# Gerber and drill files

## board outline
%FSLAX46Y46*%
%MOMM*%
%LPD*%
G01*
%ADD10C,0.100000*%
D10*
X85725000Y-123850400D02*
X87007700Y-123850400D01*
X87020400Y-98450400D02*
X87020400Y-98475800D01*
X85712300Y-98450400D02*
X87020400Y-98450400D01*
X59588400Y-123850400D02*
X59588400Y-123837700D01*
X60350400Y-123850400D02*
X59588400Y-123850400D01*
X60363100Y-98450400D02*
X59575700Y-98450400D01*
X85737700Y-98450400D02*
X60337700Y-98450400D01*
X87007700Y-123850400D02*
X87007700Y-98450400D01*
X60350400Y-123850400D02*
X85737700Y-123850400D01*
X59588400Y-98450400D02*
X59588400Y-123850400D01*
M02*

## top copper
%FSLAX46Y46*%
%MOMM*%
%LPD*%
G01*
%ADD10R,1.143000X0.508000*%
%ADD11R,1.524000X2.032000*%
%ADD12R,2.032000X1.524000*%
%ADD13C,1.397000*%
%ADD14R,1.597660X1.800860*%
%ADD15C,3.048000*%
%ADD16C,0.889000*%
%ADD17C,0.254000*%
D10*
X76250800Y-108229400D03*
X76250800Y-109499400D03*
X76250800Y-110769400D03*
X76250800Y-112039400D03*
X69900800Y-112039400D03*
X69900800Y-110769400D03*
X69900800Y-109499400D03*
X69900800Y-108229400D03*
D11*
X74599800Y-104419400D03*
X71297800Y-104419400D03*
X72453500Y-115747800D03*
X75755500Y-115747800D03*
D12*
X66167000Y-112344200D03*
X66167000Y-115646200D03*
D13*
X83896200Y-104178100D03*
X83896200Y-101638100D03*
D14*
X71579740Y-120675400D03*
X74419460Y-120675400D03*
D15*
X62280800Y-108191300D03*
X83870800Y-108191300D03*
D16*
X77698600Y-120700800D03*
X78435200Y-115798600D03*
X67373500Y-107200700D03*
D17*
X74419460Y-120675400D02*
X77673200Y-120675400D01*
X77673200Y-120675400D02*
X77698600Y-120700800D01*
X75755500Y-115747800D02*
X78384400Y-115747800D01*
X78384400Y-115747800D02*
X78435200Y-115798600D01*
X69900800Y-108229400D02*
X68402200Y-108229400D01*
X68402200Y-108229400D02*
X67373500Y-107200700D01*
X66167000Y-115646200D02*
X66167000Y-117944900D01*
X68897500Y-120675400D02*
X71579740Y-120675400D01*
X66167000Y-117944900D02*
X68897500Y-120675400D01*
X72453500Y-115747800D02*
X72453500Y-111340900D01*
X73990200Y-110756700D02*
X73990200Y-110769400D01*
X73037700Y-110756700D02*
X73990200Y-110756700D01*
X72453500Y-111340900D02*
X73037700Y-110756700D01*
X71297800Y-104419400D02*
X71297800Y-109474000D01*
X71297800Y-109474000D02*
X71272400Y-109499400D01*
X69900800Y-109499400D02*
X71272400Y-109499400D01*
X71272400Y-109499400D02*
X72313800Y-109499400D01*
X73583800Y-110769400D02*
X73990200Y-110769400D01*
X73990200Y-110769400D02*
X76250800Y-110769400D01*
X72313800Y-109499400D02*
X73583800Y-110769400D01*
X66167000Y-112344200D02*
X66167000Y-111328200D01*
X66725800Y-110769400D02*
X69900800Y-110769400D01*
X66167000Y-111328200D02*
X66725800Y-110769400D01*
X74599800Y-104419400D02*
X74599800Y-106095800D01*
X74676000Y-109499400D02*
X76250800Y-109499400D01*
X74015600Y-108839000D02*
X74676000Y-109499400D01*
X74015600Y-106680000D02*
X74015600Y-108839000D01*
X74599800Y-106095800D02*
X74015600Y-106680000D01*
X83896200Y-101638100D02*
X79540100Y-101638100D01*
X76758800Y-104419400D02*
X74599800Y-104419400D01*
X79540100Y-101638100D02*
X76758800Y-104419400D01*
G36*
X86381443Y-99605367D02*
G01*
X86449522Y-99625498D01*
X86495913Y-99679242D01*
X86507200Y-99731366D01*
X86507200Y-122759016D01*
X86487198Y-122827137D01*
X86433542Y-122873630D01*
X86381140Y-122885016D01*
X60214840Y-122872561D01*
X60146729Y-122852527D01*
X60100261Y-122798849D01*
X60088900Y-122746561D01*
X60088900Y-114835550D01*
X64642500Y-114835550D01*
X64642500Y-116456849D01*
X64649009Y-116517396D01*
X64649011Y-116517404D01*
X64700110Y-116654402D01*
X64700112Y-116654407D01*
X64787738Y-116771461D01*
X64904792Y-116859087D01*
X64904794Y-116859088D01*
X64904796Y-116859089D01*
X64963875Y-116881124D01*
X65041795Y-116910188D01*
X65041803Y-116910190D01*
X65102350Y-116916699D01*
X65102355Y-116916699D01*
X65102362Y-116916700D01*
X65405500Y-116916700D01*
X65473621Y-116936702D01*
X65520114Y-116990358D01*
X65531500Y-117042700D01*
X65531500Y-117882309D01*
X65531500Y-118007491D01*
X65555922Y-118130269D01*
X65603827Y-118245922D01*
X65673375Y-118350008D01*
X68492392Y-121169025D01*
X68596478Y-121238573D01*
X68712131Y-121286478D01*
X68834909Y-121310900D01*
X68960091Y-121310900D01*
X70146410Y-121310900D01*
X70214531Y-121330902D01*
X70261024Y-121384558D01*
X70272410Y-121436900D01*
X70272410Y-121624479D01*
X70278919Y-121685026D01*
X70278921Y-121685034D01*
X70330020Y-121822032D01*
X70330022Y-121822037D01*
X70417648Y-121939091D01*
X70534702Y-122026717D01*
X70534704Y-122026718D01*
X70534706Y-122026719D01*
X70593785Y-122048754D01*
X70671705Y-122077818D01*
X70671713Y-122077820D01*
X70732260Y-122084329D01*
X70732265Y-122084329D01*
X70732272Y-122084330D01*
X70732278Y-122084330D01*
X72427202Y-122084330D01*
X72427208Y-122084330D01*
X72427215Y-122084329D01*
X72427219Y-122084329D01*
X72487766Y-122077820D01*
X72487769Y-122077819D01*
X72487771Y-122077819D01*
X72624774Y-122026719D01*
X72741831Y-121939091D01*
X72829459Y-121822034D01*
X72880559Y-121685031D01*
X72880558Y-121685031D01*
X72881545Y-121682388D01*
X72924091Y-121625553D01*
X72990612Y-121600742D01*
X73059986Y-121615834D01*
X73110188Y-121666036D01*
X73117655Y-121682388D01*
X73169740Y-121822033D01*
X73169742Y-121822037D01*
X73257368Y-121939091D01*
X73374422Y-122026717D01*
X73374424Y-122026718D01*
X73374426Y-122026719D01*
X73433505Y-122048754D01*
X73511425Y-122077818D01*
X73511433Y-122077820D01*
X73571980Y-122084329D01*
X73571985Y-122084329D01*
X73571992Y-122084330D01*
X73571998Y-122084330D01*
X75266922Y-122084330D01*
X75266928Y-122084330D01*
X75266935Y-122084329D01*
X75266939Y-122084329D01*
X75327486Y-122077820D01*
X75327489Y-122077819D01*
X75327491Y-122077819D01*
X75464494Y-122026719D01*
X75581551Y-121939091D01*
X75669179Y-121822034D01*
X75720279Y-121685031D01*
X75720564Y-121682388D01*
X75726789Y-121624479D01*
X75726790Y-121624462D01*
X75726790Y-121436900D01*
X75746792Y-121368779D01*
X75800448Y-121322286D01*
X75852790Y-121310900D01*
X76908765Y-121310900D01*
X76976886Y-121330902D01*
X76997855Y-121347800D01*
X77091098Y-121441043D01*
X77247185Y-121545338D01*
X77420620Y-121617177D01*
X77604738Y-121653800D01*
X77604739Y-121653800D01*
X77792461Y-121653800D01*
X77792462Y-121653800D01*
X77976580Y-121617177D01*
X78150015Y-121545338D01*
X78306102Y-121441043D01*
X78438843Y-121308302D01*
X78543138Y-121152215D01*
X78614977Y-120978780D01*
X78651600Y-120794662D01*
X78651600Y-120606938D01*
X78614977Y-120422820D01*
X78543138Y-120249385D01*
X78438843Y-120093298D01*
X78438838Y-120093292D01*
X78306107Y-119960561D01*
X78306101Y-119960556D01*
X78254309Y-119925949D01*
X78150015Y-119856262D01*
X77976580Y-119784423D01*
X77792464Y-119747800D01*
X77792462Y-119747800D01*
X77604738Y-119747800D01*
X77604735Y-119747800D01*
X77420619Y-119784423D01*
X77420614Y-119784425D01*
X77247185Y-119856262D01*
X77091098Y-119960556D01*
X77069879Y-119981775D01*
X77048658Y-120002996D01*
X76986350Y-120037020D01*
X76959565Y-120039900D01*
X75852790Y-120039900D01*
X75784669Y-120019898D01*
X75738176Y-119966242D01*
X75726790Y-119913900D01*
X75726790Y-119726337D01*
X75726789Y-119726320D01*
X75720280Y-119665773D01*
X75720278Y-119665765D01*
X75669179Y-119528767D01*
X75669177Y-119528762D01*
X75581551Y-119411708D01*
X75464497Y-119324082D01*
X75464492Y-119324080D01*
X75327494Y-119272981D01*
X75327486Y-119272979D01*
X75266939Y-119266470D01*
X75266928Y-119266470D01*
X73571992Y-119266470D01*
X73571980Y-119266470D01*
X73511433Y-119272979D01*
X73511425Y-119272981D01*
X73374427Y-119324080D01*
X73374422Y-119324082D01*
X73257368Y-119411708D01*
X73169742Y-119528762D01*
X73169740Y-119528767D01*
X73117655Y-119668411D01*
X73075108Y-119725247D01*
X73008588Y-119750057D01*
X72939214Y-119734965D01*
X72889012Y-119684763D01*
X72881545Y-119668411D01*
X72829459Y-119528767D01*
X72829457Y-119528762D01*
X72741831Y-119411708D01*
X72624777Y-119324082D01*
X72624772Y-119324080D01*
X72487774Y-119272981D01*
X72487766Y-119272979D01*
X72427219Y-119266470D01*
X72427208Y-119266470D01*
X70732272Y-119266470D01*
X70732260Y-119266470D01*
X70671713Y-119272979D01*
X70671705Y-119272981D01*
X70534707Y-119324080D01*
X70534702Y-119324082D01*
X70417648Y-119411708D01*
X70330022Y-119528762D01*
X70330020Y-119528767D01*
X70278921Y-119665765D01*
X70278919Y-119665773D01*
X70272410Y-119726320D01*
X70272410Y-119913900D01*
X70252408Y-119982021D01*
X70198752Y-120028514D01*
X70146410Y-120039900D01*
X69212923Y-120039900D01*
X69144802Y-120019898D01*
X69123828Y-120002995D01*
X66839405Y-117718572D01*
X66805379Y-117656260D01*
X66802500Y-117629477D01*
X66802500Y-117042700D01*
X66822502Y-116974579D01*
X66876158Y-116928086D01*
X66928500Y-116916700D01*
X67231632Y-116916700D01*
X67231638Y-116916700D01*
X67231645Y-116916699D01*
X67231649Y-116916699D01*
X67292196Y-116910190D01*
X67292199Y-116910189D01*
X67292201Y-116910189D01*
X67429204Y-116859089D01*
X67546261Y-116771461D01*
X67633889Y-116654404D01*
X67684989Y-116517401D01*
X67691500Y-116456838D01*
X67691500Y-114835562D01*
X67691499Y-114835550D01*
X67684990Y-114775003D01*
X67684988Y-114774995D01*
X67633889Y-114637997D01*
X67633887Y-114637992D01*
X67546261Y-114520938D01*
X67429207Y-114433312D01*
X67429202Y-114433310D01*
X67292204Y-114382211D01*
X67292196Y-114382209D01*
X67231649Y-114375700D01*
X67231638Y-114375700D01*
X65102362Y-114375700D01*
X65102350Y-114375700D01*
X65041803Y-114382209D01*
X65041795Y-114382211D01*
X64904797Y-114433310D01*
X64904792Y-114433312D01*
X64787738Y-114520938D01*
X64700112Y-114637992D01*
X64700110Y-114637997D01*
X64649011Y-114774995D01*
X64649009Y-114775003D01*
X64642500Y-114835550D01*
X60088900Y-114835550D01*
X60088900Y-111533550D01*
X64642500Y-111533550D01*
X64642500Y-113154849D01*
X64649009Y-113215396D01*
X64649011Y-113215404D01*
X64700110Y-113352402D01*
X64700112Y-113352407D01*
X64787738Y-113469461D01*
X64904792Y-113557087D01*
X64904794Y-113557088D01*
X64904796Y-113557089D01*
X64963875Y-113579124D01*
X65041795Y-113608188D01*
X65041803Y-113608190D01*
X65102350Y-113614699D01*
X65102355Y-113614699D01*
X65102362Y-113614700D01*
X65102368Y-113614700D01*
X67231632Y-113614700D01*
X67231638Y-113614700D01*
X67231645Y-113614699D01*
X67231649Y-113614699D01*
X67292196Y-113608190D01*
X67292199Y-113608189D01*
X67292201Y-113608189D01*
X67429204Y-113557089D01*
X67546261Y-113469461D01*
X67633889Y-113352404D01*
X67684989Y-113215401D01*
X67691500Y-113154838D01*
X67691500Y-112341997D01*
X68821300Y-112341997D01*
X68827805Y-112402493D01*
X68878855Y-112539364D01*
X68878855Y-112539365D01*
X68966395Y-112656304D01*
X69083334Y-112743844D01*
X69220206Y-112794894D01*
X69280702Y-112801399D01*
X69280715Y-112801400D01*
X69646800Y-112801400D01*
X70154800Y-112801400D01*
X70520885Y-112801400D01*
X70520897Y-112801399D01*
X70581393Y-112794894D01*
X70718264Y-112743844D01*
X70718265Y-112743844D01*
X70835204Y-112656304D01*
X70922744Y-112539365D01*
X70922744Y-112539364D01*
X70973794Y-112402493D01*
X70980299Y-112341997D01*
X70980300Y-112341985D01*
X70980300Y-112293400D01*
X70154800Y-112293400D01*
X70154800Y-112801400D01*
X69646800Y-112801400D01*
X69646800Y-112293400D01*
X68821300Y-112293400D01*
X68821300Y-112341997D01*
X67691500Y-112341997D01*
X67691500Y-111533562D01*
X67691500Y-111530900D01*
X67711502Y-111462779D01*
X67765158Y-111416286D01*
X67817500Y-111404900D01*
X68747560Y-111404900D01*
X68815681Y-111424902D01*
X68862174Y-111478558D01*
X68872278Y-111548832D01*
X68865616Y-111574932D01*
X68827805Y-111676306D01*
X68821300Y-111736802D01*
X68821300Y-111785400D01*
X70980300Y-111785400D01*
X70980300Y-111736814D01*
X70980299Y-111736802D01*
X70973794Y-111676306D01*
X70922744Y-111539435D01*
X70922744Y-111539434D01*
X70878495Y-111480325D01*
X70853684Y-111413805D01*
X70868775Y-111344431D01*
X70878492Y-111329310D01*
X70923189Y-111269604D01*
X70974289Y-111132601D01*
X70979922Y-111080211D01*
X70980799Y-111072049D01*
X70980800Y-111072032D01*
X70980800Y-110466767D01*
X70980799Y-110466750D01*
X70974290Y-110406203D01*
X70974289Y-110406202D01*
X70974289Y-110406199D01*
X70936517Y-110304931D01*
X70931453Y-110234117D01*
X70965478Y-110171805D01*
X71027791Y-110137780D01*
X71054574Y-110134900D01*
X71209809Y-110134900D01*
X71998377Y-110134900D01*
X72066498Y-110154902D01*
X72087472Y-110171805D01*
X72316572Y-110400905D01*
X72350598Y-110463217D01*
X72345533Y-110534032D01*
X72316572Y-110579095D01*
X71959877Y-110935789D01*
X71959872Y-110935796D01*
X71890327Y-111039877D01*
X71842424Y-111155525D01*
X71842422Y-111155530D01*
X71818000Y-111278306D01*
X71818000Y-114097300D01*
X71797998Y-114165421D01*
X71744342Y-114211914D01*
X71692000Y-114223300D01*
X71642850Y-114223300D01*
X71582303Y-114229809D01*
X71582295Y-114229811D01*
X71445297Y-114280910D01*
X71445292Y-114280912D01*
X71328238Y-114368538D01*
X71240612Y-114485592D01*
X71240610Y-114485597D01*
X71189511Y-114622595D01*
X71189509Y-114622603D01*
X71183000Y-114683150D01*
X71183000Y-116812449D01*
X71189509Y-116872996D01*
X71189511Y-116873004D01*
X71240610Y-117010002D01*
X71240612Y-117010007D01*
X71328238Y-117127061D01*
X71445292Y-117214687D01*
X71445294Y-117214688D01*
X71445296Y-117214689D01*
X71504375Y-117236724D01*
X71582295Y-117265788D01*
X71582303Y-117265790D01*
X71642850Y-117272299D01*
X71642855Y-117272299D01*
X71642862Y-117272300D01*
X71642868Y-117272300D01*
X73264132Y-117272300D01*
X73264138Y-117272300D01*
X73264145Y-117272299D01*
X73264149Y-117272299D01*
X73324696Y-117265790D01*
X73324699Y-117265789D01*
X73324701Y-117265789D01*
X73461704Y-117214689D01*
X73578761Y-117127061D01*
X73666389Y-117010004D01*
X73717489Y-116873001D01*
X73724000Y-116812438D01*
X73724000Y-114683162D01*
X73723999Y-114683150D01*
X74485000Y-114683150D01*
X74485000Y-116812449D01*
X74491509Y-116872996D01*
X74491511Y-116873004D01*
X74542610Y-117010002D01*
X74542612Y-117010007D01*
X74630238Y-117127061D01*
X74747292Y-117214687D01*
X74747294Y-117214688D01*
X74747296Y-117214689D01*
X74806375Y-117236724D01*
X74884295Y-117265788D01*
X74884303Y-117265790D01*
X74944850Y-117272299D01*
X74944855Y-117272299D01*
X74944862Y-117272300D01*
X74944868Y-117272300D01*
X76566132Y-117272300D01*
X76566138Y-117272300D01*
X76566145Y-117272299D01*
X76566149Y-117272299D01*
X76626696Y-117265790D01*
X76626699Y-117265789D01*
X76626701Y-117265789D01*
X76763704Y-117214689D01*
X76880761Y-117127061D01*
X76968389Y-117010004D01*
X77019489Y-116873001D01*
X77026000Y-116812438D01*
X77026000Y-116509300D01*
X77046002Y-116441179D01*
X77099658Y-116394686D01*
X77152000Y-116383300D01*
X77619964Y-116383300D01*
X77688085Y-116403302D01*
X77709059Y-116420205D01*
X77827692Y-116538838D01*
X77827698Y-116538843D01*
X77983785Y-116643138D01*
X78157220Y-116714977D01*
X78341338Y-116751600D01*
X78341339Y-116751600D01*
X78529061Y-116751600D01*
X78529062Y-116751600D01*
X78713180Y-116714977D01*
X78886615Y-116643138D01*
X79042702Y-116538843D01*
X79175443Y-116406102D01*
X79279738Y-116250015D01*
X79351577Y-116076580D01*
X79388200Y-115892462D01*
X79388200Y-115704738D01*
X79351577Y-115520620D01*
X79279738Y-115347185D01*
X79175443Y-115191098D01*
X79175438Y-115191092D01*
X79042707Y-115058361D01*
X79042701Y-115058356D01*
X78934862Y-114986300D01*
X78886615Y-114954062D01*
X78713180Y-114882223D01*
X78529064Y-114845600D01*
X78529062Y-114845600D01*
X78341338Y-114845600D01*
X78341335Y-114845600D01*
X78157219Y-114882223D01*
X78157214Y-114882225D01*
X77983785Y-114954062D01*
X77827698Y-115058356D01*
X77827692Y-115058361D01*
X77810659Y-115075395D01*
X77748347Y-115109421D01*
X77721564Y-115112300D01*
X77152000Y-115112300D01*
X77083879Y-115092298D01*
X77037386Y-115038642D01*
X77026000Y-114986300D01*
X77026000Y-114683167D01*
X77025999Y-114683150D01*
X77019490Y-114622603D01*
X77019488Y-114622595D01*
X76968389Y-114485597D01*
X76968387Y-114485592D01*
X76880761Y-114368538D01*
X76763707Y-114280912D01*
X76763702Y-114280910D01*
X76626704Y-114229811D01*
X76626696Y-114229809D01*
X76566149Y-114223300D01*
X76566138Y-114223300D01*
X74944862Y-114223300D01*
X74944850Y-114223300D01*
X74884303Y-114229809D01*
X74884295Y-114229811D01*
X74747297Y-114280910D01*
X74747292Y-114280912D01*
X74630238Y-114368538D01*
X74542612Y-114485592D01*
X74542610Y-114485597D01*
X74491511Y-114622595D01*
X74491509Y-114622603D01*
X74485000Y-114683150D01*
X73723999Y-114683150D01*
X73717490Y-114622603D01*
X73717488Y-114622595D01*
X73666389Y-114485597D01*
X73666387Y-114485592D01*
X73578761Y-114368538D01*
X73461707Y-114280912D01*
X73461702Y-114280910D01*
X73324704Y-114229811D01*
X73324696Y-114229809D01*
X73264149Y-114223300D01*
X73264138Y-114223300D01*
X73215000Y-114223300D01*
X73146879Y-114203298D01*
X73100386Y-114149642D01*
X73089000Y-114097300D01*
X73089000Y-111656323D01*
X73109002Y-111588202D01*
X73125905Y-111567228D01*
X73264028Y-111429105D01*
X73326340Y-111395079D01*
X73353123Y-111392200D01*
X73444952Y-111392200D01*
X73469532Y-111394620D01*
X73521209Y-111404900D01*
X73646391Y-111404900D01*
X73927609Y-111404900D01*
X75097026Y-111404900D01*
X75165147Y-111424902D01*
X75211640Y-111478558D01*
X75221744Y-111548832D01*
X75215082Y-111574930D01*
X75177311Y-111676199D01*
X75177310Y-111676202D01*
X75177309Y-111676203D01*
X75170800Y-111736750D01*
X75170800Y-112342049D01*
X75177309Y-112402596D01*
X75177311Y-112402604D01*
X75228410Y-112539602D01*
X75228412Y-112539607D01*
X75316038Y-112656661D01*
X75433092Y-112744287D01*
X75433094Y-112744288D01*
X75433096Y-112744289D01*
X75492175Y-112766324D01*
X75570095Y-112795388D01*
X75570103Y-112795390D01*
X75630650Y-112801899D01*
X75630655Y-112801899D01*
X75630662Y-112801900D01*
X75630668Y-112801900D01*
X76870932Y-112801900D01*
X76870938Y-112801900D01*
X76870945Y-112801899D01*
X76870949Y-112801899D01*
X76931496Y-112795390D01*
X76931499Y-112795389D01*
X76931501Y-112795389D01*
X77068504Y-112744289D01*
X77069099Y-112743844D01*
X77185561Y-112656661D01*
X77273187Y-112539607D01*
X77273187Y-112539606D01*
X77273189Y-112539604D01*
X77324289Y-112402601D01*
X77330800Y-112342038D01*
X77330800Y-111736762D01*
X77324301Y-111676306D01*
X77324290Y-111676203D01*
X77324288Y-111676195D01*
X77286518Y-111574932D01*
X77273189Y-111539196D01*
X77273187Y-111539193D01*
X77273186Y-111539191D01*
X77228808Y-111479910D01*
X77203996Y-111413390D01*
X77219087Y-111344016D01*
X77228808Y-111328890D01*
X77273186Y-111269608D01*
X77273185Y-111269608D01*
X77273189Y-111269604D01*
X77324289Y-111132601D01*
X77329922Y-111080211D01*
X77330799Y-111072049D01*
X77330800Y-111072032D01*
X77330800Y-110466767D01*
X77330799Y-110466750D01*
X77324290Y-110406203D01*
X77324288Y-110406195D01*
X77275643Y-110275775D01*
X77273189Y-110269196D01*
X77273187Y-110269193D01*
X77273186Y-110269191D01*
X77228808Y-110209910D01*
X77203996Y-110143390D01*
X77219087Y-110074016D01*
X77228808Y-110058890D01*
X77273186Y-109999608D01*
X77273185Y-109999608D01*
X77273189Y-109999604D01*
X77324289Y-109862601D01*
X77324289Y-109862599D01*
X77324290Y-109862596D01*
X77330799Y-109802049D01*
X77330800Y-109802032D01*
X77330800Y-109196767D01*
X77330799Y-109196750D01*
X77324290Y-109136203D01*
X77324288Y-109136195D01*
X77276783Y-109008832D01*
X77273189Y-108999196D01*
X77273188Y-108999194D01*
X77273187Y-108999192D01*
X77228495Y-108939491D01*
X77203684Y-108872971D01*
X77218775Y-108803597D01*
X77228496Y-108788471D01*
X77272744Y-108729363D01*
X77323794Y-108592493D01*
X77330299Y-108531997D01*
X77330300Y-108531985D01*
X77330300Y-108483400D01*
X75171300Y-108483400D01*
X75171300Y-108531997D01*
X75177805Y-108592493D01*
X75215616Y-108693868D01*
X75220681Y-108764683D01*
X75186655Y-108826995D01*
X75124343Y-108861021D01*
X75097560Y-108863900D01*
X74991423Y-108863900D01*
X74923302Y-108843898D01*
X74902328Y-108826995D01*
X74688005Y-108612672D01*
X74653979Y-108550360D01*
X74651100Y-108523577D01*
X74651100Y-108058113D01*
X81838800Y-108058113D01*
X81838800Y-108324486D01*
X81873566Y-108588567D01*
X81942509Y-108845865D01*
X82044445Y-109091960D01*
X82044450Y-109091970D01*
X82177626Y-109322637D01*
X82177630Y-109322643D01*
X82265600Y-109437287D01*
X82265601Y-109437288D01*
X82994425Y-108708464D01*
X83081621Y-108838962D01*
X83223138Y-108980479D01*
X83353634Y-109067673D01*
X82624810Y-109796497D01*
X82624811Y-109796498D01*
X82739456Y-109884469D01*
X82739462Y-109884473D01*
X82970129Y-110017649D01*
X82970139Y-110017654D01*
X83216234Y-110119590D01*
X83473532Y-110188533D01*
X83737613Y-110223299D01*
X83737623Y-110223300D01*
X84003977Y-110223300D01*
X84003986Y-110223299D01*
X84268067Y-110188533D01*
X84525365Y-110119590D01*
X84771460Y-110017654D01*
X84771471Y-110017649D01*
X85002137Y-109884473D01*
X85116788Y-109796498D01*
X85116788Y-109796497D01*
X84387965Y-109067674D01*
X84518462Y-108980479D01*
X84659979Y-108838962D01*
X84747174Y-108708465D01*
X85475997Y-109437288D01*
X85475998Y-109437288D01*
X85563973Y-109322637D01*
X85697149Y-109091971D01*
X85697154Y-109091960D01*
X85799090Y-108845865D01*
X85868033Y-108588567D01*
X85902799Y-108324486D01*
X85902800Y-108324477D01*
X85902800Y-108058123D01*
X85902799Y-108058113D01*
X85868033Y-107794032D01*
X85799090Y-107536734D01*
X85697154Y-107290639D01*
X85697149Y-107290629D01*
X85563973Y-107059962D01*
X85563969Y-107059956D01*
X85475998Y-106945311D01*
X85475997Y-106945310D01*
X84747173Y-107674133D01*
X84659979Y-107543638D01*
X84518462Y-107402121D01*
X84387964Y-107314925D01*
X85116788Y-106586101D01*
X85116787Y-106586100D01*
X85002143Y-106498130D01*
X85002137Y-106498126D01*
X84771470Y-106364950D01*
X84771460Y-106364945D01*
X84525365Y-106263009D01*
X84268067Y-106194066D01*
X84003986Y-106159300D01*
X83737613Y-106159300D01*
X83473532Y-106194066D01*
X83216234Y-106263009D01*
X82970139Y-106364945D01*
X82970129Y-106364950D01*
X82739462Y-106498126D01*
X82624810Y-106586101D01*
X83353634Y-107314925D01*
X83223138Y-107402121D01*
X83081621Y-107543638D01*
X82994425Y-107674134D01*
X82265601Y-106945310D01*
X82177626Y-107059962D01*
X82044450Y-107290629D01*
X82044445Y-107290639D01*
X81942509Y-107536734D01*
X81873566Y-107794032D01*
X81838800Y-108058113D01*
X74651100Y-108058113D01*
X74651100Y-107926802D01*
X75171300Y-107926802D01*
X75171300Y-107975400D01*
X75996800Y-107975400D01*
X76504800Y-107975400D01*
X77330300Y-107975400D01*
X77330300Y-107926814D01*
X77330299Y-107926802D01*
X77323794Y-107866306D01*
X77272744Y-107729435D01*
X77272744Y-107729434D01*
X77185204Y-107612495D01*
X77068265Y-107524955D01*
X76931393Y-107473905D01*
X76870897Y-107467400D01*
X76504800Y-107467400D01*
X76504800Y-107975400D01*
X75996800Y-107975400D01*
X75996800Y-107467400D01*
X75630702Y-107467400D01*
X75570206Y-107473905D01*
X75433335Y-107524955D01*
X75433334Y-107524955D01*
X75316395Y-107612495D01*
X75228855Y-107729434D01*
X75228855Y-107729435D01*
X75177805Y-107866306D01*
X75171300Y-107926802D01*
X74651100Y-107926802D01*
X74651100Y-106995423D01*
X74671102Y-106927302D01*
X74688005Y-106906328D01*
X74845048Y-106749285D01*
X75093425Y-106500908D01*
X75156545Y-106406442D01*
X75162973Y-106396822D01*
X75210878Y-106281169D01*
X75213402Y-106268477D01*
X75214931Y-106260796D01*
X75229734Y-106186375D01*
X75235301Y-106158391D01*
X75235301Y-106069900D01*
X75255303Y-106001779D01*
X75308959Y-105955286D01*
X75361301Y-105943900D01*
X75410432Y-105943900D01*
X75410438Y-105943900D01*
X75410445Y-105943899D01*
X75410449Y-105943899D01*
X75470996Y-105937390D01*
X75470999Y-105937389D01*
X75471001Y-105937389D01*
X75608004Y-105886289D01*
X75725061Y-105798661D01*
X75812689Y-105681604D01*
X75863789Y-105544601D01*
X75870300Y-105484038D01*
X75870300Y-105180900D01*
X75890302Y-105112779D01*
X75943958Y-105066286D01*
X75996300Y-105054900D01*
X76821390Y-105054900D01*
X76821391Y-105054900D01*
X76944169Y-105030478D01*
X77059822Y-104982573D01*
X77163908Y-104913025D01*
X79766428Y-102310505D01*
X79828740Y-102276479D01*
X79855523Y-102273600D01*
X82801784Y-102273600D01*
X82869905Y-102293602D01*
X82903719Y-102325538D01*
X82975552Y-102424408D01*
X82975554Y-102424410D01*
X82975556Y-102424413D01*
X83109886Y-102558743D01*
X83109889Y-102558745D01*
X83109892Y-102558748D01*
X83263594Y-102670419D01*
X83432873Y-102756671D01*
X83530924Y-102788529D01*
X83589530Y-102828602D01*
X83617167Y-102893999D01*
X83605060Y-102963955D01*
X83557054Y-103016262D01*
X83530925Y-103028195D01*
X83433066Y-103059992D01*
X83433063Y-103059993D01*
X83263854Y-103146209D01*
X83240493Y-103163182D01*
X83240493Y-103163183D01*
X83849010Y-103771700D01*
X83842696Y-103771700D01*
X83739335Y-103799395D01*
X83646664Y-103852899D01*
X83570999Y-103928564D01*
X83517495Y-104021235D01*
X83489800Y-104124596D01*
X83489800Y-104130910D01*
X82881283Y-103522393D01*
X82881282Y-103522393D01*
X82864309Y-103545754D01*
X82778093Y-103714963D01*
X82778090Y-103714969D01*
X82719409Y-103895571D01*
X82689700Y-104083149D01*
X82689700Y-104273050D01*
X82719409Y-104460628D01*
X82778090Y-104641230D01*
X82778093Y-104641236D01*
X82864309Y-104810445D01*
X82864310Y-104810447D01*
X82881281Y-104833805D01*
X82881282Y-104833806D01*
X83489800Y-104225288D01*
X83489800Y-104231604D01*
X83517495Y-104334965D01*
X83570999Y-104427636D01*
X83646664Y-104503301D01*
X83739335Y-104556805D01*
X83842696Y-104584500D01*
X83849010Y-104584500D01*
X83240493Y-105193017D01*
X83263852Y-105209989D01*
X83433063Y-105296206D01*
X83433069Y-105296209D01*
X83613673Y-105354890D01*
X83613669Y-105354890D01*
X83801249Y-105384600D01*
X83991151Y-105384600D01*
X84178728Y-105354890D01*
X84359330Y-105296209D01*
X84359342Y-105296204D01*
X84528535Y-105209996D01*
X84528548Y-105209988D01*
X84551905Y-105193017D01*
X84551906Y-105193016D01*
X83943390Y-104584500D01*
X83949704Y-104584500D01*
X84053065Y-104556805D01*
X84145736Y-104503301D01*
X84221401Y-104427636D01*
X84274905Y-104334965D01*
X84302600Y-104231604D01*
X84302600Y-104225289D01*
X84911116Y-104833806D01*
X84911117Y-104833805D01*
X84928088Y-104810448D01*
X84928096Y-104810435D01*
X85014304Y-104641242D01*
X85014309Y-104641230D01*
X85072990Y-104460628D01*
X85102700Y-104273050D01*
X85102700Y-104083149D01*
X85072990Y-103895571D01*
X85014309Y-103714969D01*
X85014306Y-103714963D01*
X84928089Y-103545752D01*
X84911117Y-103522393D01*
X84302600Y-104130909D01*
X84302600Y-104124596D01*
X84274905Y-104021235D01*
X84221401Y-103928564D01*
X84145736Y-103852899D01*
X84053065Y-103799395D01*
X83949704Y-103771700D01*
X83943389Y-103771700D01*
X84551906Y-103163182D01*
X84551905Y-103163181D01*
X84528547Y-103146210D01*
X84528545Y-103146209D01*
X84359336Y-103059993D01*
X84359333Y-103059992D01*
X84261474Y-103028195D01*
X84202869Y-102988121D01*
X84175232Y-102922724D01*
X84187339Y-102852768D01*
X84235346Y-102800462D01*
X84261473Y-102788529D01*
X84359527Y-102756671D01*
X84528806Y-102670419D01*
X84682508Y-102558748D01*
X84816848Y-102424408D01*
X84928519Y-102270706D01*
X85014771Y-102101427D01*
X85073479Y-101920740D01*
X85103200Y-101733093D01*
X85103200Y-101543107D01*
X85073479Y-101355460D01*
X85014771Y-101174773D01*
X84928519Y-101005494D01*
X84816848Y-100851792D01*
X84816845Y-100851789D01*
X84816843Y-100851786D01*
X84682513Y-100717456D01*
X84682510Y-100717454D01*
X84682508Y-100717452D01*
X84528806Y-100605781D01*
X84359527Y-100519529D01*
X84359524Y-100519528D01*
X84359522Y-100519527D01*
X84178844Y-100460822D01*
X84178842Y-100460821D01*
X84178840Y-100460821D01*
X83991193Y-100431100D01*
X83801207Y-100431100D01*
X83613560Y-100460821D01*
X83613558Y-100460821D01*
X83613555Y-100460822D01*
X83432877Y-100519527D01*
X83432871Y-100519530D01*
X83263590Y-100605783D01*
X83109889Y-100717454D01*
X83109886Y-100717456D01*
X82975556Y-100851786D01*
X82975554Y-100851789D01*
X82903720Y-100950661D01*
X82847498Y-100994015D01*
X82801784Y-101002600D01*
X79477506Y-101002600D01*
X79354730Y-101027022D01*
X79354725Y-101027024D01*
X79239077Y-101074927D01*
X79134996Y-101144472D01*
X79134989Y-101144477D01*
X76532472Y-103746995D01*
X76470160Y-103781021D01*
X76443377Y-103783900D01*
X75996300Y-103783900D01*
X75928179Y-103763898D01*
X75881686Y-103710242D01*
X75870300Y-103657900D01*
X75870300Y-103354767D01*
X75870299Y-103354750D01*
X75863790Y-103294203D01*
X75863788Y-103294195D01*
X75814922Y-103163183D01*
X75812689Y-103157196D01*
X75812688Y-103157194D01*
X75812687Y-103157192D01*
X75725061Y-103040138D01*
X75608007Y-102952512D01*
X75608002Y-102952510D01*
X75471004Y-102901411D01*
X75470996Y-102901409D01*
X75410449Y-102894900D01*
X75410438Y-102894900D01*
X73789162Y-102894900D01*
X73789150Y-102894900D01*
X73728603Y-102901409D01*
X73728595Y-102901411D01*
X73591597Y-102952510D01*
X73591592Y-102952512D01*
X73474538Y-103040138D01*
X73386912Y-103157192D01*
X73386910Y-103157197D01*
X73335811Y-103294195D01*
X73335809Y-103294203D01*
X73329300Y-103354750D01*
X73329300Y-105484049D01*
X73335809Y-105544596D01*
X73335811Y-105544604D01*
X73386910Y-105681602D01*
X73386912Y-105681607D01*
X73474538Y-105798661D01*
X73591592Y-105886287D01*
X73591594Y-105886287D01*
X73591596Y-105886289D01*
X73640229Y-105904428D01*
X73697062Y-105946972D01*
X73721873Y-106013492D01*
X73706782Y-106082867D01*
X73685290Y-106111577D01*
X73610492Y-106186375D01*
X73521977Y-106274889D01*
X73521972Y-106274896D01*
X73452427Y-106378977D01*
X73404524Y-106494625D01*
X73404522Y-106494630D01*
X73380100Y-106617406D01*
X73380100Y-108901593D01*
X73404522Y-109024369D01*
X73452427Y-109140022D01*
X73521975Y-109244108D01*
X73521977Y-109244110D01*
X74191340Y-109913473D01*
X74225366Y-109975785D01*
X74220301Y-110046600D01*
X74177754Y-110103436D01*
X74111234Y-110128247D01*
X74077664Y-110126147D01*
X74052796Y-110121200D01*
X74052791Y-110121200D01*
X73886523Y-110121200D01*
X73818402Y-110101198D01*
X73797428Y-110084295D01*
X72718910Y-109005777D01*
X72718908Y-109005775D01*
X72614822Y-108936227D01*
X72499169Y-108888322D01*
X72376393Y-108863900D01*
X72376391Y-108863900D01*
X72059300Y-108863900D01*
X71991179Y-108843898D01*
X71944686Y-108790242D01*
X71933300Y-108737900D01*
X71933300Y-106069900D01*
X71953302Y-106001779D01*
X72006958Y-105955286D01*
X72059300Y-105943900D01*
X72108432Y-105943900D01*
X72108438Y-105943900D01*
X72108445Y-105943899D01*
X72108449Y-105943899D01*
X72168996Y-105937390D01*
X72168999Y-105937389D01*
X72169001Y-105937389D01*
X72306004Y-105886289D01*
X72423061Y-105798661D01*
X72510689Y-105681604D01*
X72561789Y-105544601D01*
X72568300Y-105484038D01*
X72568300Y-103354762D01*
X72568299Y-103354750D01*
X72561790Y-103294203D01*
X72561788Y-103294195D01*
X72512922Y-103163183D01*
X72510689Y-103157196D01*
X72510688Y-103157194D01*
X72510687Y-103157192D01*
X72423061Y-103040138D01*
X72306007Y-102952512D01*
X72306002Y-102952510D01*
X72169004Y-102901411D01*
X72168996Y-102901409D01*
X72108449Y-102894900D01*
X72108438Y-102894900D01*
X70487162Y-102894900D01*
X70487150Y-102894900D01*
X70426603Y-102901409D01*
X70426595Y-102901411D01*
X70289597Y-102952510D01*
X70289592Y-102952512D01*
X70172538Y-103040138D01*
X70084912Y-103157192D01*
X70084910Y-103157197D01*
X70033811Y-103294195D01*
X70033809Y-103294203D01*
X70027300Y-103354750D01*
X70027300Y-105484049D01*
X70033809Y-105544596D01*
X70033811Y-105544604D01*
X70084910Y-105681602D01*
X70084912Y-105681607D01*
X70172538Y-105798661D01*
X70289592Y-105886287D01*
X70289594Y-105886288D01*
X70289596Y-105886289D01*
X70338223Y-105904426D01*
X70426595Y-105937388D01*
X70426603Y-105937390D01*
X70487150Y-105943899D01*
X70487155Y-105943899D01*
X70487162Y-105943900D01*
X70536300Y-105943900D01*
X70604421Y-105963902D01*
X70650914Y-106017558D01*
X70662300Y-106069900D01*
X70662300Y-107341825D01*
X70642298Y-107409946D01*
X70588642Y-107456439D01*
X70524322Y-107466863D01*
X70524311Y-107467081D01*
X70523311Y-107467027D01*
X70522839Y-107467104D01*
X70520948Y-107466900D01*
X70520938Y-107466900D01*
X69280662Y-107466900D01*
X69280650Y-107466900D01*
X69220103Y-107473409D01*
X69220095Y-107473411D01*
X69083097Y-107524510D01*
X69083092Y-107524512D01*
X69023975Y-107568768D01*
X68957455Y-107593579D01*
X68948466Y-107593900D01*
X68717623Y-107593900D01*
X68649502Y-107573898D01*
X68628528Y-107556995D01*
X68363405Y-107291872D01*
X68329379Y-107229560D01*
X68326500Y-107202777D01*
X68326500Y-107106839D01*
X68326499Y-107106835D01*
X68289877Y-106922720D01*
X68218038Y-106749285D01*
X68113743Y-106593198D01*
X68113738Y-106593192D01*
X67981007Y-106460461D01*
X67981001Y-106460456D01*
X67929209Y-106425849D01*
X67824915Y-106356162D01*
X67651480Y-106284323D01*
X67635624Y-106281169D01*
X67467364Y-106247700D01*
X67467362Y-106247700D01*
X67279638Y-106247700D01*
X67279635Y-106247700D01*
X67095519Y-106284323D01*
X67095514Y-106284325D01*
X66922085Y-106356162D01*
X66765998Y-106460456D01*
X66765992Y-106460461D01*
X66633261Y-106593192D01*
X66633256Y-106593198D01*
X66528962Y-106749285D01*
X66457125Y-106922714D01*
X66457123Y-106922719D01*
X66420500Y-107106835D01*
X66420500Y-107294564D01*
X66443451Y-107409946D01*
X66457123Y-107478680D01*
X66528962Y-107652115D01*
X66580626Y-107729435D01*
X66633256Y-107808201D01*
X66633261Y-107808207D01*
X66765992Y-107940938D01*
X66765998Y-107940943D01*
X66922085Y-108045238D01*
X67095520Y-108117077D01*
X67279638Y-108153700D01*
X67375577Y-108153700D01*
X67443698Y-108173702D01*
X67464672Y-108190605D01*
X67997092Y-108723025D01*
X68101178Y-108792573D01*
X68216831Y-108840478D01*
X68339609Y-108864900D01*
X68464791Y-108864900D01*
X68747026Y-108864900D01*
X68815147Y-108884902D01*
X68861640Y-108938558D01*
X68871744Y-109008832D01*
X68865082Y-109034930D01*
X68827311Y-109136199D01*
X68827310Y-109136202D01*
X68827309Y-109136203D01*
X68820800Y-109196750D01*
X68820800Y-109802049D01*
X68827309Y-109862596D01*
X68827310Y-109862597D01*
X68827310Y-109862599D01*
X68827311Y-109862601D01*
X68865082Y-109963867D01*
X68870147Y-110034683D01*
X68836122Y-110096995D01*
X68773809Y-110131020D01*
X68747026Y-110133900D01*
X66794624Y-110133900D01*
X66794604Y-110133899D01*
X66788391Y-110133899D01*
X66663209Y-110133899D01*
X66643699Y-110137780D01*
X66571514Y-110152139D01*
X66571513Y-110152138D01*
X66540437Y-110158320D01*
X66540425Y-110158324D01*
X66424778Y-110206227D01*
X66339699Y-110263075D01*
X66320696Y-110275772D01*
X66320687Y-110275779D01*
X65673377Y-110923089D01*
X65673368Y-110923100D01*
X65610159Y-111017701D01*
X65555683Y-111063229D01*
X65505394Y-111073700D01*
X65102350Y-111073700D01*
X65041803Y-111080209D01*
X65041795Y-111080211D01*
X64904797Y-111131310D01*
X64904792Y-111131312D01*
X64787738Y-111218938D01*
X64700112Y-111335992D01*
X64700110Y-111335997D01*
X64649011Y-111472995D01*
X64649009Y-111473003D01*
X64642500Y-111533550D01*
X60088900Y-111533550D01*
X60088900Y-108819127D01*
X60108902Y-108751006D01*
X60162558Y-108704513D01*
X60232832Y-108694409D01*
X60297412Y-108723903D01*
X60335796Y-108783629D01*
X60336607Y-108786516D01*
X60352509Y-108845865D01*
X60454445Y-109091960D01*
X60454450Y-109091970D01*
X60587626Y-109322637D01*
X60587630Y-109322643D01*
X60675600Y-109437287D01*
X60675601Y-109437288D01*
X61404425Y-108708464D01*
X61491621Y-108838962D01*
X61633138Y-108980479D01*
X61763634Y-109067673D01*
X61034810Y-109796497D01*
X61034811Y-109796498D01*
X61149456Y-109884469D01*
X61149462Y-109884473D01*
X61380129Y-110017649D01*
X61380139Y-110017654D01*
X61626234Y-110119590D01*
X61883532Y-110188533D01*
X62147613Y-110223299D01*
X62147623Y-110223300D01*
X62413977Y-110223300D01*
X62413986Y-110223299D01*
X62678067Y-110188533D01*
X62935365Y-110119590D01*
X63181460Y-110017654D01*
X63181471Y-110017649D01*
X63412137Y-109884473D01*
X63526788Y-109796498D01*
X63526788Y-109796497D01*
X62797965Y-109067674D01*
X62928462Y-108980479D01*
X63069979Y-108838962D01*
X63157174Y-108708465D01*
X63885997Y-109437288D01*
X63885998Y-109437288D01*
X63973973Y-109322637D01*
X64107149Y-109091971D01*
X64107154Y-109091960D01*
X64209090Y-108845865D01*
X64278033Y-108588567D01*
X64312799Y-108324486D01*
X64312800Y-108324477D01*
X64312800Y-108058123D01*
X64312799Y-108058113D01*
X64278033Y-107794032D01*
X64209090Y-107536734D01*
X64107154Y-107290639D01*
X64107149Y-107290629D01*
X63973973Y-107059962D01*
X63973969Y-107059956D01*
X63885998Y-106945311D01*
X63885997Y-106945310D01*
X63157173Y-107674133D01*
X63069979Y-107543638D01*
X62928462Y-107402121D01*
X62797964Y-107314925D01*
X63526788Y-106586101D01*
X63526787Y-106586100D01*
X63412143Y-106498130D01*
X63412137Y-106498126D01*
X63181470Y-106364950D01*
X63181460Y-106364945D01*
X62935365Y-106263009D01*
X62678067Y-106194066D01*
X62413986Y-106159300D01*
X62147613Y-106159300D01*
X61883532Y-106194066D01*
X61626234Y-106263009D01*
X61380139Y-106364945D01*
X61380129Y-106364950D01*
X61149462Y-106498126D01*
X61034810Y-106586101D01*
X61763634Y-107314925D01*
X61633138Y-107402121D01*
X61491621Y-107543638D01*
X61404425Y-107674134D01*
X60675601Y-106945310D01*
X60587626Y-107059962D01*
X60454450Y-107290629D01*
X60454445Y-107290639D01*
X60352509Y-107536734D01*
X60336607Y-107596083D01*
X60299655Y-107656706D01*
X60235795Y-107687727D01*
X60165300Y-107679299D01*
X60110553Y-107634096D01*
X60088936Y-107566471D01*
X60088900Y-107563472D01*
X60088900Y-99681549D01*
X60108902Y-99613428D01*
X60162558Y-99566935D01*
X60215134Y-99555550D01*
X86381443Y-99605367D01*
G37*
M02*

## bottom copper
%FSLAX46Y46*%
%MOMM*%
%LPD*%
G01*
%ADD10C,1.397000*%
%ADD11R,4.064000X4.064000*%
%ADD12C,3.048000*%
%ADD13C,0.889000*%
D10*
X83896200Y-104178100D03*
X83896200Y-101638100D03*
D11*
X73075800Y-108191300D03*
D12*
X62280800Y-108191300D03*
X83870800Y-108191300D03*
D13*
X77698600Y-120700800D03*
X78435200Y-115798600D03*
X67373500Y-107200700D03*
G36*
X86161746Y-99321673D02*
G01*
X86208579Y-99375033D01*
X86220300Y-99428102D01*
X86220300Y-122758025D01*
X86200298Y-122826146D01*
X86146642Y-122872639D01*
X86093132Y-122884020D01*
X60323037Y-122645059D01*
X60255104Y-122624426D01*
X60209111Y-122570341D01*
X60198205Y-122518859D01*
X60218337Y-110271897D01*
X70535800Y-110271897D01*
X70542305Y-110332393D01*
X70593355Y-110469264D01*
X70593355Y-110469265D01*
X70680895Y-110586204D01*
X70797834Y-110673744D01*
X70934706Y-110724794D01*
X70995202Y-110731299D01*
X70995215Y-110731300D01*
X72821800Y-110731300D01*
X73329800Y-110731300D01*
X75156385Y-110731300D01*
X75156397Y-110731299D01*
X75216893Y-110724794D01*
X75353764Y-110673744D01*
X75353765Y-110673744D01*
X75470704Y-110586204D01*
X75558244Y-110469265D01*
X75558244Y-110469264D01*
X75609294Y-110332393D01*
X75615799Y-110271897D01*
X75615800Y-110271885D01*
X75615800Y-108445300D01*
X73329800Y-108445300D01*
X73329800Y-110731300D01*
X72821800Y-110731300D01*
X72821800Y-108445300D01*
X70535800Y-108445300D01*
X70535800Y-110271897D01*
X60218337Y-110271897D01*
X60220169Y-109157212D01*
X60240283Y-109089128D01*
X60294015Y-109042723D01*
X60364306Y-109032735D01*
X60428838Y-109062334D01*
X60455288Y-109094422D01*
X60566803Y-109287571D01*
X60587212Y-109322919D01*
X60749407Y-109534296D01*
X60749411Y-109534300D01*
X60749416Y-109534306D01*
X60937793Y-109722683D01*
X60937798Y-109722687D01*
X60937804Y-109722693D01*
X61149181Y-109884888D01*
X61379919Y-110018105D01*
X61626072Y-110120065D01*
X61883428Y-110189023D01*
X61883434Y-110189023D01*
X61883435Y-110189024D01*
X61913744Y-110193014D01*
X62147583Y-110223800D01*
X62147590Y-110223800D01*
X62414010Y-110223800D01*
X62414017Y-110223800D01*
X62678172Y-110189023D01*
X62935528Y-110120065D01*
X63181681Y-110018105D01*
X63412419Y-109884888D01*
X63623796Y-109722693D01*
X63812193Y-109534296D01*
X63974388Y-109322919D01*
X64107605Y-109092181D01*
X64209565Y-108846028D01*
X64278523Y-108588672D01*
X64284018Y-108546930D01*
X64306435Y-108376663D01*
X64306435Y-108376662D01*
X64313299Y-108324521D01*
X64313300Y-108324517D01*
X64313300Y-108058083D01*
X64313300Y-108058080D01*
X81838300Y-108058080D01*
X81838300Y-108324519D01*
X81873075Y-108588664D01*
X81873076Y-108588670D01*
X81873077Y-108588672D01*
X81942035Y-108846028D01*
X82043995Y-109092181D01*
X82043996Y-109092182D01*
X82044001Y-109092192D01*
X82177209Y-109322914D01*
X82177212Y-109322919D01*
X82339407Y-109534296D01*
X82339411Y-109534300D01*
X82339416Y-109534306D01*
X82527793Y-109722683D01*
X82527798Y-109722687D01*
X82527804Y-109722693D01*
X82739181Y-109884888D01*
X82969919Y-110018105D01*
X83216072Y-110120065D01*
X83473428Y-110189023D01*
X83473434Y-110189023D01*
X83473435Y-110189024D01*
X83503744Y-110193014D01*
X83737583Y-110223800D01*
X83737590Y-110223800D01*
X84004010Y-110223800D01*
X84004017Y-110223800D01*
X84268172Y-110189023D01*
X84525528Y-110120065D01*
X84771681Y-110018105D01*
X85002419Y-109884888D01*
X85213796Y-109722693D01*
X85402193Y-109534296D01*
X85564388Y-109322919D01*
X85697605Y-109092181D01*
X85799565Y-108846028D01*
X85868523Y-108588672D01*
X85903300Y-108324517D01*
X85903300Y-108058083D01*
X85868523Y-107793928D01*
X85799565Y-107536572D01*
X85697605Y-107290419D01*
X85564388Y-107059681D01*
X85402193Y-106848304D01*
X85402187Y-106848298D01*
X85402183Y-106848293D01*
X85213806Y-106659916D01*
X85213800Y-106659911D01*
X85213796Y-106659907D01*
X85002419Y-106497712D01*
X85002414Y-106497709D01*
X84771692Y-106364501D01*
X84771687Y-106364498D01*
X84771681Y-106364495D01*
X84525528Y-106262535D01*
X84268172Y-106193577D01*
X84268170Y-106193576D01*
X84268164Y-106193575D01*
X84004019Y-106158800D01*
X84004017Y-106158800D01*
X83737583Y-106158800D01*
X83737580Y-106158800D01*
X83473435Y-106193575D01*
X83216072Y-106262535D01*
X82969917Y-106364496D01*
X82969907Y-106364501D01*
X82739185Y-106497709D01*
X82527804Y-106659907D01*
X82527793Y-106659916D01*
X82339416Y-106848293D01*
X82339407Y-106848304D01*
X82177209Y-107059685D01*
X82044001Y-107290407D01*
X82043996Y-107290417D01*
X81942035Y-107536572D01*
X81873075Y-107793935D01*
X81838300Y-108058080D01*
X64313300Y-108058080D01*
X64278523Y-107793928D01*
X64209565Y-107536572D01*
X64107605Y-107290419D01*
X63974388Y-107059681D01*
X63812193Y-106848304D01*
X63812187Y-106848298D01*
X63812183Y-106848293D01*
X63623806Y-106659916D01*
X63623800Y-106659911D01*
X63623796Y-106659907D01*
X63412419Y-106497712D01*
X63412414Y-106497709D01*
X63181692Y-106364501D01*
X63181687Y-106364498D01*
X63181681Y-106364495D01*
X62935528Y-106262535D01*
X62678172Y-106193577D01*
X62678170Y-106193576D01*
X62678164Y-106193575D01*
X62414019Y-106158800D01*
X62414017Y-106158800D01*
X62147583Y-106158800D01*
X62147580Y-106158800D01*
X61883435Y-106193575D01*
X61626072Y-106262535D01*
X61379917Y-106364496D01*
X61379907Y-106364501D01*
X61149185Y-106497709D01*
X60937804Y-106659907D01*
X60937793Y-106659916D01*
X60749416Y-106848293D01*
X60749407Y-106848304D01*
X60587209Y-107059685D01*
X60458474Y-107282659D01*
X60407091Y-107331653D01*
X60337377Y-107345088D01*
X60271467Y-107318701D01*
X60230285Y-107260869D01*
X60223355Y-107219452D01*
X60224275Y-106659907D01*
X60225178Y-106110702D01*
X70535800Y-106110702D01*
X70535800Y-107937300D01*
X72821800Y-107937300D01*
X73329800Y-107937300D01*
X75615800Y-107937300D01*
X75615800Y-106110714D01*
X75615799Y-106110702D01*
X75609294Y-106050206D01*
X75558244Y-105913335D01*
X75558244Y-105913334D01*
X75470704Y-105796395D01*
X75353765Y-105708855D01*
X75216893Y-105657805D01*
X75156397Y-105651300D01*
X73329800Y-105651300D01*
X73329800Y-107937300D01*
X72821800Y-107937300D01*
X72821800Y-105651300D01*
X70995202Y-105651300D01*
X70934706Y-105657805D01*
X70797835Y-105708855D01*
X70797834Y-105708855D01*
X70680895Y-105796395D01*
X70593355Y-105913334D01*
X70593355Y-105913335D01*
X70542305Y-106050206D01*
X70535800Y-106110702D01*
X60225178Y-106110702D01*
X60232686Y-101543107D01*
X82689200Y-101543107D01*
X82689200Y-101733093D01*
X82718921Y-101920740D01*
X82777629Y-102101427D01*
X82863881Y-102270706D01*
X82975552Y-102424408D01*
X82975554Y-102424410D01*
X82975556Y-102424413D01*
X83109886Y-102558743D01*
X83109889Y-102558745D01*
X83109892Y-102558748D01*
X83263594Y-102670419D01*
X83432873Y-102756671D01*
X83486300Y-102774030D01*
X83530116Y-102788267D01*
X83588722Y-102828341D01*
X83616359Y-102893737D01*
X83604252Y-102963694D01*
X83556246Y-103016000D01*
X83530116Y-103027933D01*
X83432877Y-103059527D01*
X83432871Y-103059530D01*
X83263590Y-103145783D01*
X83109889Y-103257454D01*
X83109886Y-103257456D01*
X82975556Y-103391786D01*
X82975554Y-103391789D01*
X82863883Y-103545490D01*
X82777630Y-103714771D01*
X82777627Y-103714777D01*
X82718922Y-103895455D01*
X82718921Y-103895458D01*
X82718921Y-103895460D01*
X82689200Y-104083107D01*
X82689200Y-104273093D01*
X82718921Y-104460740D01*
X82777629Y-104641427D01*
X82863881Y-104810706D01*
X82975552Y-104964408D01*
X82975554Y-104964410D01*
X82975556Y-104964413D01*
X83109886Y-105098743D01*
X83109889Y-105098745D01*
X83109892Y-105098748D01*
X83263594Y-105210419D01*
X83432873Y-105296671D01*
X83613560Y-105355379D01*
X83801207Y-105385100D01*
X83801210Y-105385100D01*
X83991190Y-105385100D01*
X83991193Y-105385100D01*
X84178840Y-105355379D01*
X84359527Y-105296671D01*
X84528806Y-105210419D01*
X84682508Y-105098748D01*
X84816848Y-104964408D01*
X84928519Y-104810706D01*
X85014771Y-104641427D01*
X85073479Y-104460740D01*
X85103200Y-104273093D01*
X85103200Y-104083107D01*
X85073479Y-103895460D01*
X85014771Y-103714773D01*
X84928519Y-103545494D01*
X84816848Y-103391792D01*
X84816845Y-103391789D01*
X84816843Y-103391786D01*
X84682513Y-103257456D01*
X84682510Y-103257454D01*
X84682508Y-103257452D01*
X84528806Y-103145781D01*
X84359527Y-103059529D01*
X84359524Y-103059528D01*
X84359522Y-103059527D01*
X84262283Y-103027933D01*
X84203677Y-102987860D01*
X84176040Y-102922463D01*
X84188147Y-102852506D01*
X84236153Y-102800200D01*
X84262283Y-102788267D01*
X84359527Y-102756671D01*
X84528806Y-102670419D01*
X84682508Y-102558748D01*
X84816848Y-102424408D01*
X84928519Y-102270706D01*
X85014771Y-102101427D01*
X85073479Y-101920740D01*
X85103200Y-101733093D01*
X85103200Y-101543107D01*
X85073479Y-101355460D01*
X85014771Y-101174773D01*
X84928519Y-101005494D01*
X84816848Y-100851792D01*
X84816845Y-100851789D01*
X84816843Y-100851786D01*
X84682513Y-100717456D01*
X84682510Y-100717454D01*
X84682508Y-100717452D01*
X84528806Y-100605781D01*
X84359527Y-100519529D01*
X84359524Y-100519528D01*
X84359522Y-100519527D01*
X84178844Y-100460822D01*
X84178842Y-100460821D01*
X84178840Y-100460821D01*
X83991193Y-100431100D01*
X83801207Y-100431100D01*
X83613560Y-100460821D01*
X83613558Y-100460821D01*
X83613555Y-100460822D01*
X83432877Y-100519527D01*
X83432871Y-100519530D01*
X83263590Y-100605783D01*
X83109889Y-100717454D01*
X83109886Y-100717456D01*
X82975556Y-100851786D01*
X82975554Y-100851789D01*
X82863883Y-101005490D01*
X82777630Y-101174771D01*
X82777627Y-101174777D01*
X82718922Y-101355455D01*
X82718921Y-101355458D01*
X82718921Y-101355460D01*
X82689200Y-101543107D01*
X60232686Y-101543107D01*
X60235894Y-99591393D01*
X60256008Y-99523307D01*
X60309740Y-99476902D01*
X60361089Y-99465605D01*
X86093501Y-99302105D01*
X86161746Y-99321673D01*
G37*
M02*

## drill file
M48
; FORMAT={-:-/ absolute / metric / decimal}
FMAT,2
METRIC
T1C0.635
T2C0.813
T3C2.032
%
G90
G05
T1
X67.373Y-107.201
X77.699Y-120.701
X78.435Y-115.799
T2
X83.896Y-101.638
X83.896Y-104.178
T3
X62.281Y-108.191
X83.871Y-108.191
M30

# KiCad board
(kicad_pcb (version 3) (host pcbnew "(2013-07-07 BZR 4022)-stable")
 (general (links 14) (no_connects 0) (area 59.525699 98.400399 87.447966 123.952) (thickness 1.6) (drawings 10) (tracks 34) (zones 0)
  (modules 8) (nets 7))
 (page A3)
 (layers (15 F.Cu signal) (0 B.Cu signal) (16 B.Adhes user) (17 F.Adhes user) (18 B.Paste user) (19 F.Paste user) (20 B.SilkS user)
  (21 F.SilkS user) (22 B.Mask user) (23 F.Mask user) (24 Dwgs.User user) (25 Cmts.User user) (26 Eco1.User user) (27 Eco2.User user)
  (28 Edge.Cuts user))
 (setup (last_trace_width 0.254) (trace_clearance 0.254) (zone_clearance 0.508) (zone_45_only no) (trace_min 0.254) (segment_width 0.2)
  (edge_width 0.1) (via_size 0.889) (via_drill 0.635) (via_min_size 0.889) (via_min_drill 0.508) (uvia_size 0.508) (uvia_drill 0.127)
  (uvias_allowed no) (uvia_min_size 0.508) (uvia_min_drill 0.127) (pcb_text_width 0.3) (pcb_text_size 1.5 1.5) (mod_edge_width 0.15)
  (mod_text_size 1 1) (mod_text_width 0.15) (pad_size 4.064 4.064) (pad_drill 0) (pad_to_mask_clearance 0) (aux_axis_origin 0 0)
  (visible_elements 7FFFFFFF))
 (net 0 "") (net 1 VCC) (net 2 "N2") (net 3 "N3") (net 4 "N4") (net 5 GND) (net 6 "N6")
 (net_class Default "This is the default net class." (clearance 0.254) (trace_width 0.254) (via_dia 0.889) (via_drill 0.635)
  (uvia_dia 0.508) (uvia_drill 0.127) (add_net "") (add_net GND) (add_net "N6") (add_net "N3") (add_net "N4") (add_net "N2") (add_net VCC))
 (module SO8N (layer F.Cu) (at 73.0758 110.1344 270)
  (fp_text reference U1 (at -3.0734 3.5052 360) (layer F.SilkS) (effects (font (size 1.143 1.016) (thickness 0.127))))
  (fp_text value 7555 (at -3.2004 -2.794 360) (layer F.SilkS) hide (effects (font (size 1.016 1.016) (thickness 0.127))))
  (pad 8 smd rect (at -1.905 -3.175 270) (size 0.508 1.143) (layers F.Cu F.Paste F.Mask) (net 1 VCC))
  (pad 7 smd rect (at -0.635 -3.175 270) (size 0.508 1.143) (layers F.Cu F.Paste F.Mask) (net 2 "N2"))
  (pad 6 smd rect (at 0.635 -3.175 270) (size 0.508 1.143) (layers F.Cu F.Paste F.Mask) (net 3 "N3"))
  (pad 5 smd rect (at 1.905 -3.175 270) (size 0.508 1.143) (layers F.Cu F.Paste F.Mask))
  (pad 4 smd rect (at 1.905 3.175 270) (size 0.508 1.143) (layers F.Cu F.Paste F.Mask) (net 1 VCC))
  (pad 3 smd rect (at 0.635 3.175 270) (size 0.508 1.143) (layers F.Cu F.Paste F.Mask) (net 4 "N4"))
  (pad 2 smd rect (at -0.635 3.175 270) (size 0.508 1.143) (layers F.Cu F.Paste F.Mask) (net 3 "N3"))
  (pad 1 smd rect (at -1.905 3.175 270) (size 0.508 1.143) (layers F.Cu F.Paste F.Mask) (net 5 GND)))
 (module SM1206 (layer F.Cu) (at 72.9488 104.4194 180)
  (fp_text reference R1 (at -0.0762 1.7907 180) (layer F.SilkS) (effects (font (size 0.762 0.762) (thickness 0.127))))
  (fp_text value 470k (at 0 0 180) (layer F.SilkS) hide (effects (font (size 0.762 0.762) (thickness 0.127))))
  (pad 1 smd rect (at -1.651 0 180) (size 1.524 2.032) (layers F.Cu F.Paste F.Mask) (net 2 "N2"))
  (pad 2 smd rect (at 1.651 0 180) (size 1.524 2.032) (layers F.Cu F.Paste F.Mask) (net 3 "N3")))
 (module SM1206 (layer F.Cu) (at 74.1045 115.7478)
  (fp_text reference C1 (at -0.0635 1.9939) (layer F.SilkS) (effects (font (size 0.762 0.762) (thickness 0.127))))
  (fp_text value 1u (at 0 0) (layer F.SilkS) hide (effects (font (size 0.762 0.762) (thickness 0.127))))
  (pad 1 smd rect (at -1.651 0) (size 1.524 2.032) (layers F.Cu F.Paste F.Mask) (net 3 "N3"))
  (pad 2 smd rect (at 1.651 0) (size 1.524 2.032) (layers F.Cu F.Paste F.Mask) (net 5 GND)))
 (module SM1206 (layer F.Cu) (at 66.167 113.9952 270)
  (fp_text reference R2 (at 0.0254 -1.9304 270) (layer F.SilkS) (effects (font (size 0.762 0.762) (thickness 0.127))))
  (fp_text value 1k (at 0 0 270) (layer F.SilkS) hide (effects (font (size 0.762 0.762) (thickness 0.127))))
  (pad 1 smd rect (at -1.651 0 270) (size 1.524 2.032) (layers F.Cu F.Paste F.Mask) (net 4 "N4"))
  (pad 2 smd rect (at 1.651 0 270) (size 1.524 2.032) (layers F.Cu F.Paste F.Mask) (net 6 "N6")))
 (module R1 (layer F.Cu) (at 83.8962 102.9081 90) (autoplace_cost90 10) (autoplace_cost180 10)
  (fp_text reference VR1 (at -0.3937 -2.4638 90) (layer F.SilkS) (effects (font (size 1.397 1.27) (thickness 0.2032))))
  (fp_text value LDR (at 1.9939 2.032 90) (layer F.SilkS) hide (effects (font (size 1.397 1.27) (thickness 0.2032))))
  (pad 1 thru_hole circle (at -1.27 0 90) (size 1.397 1.397) (drill 0.8128) (layers *.Cu *.Mask F.SilkS) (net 1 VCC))
  (pad 2 thru_hole circle (at 1.27 0 90) (size 1.397 1.397) (drill 0.8128) (layers *.Cu *.Mask F.SilkS) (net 2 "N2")))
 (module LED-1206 (layer F.Cu) (at 72.9996 120.6754)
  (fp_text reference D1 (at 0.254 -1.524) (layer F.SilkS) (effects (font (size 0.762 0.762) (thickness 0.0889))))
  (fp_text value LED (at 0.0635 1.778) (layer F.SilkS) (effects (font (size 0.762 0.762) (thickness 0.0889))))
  (pad 1 smd rect (at -1.41986 0) (size 1.59766 1.80086) (layers F.Cu F.Paste F.Mask) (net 6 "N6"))
  (pad 2 smd rect (at 1.41986 0) (size 1.59766 1.80086) (layers F.Cu F.Paste F.Mask) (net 5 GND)))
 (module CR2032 (layer B.Cu) (at 73.0758 108.1913 180)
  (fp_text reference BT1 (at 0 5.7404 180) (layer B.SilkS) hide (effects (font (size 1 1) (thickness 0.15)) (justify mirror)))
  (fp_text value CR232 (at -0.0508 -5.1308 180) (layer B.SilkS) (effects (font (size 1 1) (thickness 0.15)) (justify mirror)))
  (pad 2 smd rect (at 0 0 180) (size 4.064 4.064) (layers B.Cu B.Paste B.Mask) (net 5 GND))
  (pad 1 thru_hole circle (at 10.795 0 180) (size 3.048 3.048) (drill 2.032) (layers *.Cu *.Mask B.SilkS) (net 1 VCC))
  (pad 1 thru_hole circle (at -10.795 0 180) (size 3.048 3.048) (drill 2.032) (layers *.Cu *.Mask B.SilkS) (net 1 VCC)))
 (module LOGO (layer F.Cu) (at 83.5914 120.3706)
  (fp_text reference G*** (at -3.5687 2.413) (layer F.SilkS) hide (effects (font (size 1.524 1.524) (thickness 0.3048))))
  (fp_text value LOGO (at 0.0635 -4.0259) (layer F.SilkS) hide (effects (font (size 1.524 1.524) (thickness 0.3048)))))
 (gr_line (start 85.725 123.8504) (end 87.0077 123.8504) (angle 90) (layer Edge.Cuts) (width 0.1))
 (gr_line (start 87.0204 98.4504) (end 87.0204 98.4758) (angle 90) (layer Edge.Cuts) (width 0.1))
 (gr_line (start 85.7123 98.4504) (end 87.0204 98.4504) (angle 90) (layer Edge.Cuts) (width 0.1))
 (gr_line (start 59.5884 123.8504) (end 59.5884 123.8377) (angle 90) (layer Edge.Cuts) (width 0.1))
 (gr_line (start 60.3504 123.8504) (end 59.5884 123.8504) (angle 90) (layer Edge.Cuts) (width 0.1))
 (gr_line (start 60.3631 98.4504) (end 59.5757 98.4504) (angle 90) (layer Edge.Cuts) (width 0.1))
 (gr_line (start 85.7377 98.4504) (end 60.3377 98.4504) (angle 90) (layer Edge.Cuts) (width 0.1))
 (gr_line (start 87.0077 123.8504) (end 87.0077 98.4504) (angle 90) (layer Edge.Cuts) (width 0.1))
 (gr_line (start 60.3504 123.8504) (end 85.7377 123.8504) (angle 90) (layer Edge.Cuts) (width 0.1))
 (gr_line (start 59.5884 98.4504) (end 59.5884 123.8504) (angle 90) (layer Edge.Cuts) (width 0.1))
 (segment (start 74.41946 120.6754) (end 77.6732 120.6754) (width 0.254) (layer F.Cu) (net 5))
 (via (at 77.6986 120.7008) (size 0.889) (layers F.Cu B.Cu) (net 5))
 (segment (start 77.6732 120.6754) (end 77.6986 120.7008) (width 0.254) (layer F.Cu) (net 5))
 (segment (start 75.7555 115.7478) (end 78.3844 115.7478) (width 0.254) (layer F.Cu) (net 5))
 (via (at 78.4352 115.7986) (size 0.889) (layers F.Cu B.Cu) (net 5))
 (segment (start 78.3844 115.7478) (end 78.4352 115.7986) (width 0.254) (layer F.Cu) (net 5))
 (segment (start 69.9008 108.2294) (end 68.4022 108.2294) (width 0.254) (layer F.Cu) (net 5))
 (via (at 67.3735 107.2007) (size 0.889) (layers F.Cu B.Cu) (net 5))
 (segment (start 68.4022 108.2294) (end 67.3735 107.2007) (width 0.254) (layer F.Cu) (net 5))
 (segment (start 66.167 115.6462) (end 66.167 117.9449) (width 0.254) (layer F.Cu) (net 6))
 (segment (start 68.8975 120.6754) (end 71.57974 120.6754) (width 0.254) (layer F.Cu) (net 6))
 (segment (start 66.167 117.9449) (end 68.8975 120.6754) (width 0.254) (layer F.Cu) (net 6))
 (segment (start 72.4535 115.7478) (end 72.4535 111.3409) (width 0.254) (layer F.Cu) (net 3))
 (segment (start 73.9902 110.7567) (end 73.9902 110.7694) (width 0.254) (layer F.Cu) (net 3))
 (segment (start 73.0377 110.7567) (end 73.9902 110.7567) (width 0.254) (layer F.Cu) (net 3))
 (segment (start 72.4535 111.3409) (end 73.0377 110.7567) (width 0.254) (layer F.Cu) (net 3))
 (segment (start 71.2978 104.4194) (end 71.2978 109.474) (width 0.254) (layer F.Cu) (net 3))
 (segment (start 71.2978 109.474) (end 71.2724 109.4994) (width 0.254) (layer F.Cu) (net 3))
 (segment (start 69.9008 109.4994) (end 71.2724 109.4994) (width 0.254) (layer F.Cu) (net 3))
 (segment (start 71.2724 109.4994) (end 72.3138 109.4994) (width 0.254) (layer F.Cu) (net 3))
 (segment (start 73.5838 110.7694) (end 73.9902 110.7694) (width 0.254) (layer F.Cu) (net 3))
 (segment (start 73.9902 110.7694) (end 76.2508 110.7694) (width 0.254) (layer F.Cu) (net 3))
 (segment (start 72.3138 109.4994) (end 73.5838 110.7694) (width 0.254) (layer F.Cu) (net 3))
 (segment (start 66.167 112.3442) (end 66.167 111.3282) (width 0.254) (layer F.Cu) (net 4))
 (segment (start 66.7258 110.7694) (end 69.9008 110.7694) (width 0.254) (layer F.Cu) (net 4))
 (segment (start 66.167 111.3282) (end 66.7258 110.7694) (width 0.254) (layer F.Cu) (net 4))
 (segment (start 74.5998 104.4194) (end 74.5998 106.0958) (width 0.254) (layer F.Cu) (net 2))
 (segment (start 74.676 109.4994) (end 76.2508 109.4994) (width 0.254) (layer F.Cu) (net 2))
 (segment (start 74.0156 108.839) (end 74.676 109.4994) (width 0.254) (layer F.Cu) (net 2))
 (segment (start 74.0156 106.68) (end 74.0156 108.839) (width 0.254) (layer F.Cu) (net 2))
 (segment (start 74.5998 106.0958) (end 74.0156 106.68) (width 0.254) (layer F.Cu) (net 2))
 (segment (start 83.8962 101.6381) (end 79.5401 101.6381) (width 0.254) (layer F.Cu) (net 2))
 (segment (start 76.7588 104.4194) (end 74.5998 104.4194) (width 0.254) (layer F.Cu) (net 2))
 (segment (start 79.5401 101.6381) (end 76.7588 104.4194) (width 0.254) (layer F.Cu) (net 2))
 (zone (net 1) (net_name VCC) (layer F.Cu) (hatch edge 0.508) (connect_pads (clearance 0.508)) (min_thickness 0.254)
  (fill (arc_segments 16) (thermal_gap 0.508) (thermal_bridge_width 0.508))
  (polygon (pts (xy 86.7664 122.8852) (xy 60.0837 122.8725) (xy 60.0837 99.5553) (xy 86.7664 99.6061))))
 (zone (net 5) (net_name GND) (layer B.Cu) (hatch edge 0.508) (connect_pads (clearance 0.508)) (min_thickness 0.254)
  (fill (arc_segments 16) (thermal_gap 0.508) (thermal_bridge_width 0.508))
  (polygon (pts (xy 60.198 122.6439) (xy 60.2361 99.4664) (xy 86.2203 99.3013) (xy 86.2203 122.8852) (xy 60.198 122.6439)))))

